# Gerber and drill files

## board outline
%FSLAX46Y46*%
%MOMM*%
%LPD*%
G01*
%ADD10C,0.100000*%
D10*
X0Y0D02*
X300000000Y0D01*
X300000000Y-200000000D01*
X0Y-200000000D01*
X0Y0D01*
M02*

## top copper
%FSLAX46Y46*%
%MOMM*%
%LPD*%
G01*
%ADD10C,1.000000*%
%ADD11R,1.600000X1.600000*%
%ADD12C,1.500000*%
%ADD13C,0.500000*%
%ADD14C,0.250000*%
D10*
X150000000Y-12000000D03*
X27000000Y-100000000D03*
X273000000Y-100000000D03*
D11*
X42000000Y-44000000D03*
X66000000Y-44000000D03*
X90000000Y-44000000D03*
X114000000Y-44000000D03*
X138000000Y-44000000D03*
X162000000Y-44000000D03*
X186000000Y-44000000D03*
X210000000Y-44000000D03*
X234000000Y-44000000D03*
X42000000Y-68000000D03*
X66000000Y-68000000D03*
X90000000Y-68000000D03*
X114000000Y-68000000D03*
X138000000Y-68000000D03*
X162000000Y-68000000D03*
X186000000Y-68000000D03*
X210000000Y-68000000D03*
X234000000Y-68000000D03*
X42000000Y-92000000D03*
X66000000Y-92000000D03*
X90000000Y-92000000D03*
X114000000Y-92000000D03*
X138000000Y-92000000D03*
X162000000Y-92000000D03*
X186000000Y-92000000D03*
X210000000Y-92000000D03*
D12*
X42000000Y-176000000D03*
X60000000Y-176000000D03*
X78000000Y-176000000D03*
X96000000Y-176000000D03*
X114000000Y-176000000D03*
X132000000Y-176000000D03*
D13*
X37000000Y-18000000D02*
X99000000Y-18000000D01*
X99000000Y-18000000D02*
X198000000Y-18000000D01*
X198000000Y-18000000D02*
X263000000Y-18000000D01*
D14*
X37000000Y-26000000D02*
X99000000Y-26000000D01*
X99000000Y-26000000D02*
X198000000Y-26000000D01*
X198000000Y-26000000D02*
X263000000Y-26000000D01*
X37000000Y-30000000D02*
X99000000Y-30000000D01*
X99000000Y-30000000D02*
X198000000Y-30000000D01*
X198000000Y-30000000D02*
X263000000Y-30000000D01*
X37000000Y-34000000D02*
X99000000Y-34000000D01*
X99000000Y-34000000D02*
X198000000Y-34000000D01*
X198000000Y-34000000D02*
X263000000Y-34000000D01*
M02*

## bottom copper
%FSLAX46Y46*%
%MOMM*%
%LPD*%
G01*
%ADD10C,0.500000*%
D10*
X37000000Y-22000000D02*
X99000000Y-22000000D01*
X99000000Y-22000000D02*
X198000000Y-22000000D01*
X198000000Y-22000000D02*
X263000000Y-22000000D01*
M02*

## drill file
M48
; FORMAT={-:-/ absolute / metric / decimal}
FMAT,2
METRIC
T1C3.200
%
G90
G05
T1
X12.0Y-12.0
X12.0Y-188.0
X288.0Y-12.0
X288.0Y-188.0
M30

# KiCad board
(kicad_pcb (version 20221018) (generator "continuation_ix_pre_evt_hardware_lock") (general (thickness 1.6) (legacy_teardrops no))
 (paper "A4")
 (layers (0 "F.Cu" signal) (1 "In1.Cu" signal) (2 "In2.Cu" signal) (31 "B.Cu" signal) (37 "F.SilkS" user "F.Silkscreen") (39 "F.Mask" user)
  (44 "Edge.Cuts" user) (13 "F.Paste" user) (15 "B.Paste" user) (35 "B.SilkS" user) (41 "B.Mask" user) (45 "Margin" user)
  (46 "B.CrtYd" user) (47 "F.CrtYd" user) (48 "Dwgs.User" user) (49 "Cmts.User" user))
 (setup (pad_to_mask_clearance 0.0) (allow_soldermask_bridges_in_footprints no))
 (gr_rect (start 0 0) (end 300.0 200.0) (stroke (width 0.1) (type default)) (fill none) (layer "Edge.Cuts"))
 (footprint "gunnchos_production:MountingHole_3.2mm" (layer "F.Cu") (at 12.0 12.0)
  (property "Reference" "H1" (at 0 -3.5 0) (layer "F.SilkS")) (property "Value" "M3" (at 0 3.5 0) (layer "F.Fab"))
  (pad "" np_thru_hole circle (at 0 0) (size 3.2 3.2) (drill 3.2) (layers "*.Cu" "*.Mask")))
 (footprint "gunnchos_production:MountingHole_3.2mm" (layer "F.Cu") (at 288.0 12.0)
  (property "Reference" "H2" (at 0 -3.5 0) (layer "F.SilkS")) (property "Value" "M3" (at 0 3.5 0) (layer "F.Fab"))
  (pad "" np_thru_hole circle (at 0 0) (size 3.2 3.2) (drill 3.2) (layers "*.Cu" "*.Mask")))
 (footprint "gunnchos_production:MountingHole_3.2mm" (layer "F.Cu") (at 12.0 188.0)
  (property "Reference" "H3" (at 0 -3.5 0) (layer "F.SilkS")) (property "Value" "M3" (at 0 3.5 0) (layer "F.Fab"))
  (pad "" np_thru_hole circle (at 0 0) (size 3.2 3.2) (drill 3.2) (layers "*.Cu" "*.Mask")))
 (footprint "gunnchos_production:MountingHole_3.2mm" (layer "F.Cu") (at 288.0 188.0)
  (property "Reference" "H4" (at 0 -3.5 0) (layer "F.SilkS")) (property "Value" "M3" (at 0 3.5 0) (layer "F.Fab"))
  (pad "" np_thru_hole circle (at 0 0) (size 3.2 3.2) (drill 3.2) (layers "*.Cu" "*.Mask")))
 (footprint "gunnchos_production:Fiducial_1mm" (layer "F.Cu") (at 150.0 12.0)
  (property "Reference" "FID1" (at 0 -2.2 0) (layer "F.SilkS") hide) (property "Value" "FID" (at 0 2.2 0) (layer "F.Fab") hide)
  (pad "1" smd circle (at 0 0) (size 1 1) (layers "F.Cu") (solder_mask_margin 0.5)))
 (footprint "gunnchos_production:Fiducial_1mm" (layer "F.Cu") (at 27.0 100.0)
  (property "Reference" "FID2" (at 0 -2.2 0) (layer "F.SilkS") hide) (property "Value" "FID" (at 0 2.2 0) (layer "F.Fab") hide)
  (pad "1" smd circle (at 0 0) (size 1 1) (layers "F.Cu") (solder_mask_margin 0.5)))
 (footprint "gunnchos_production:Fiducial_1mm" (layer "F.Cu") (at 273.0 100.0)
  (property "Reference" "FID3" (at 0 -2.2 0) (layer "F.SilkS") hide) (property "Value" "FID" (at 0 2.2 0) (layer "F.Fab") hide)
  (pad "1" smd circle (at 0 0) (size 1 1) (layers "F.Cu") (solder_mask_margin 0.5)))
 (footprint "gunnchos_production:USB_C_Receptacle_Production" (layer "F.Cu") (at 42.00 44.00)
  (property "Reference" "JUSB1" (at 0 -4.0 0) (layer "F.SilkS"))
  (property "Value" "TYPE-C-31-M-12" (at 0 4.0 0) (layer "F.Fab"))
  (pad "1" smd rect (at 0 0) (size 1.6 1.6) (layers "F.Cu" "F.Paste" "F.Mask")))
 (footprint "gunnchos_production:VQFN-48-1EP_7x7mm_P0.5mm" (layer "F.Cu") (at 66.00 44.00)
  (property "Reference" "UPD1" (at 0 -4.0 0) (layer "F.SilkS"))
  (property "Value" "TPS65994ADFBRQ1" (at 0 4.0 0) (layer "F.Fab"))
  (pad "1" smd rect (at 0 0) (size 1.6 1.6) (layers "F.Cu" "F.Paste" "F.Mask")))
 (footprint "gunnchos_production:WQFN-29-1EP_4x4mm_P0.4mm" (layer "F.Cu") (at 90.00 44.00)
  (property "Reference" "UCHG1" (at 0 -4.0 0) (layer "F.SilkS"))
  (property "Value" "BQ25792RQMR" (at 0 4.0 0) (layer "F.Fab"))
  (pad "1" smd rect (at 0 0) (size 1.6 1.6) (layers "F.Cu" "F.Paste" "F.Mask")))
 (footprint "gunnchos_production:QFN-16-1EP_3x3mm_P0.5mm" (layer "F.Cu") (at 114.00 44.00)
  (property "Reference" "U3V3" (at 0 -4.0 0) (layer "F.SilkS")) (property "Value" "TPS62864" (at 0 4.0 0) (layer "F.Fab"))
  (pad "1" smd rect (at 0 0) (size 1.6 1.6) (layers "F.Cu" "F.Paste" "F.Mask")))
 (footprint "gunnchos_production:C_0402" (layer "F.Cu") (at 138.00 44.00) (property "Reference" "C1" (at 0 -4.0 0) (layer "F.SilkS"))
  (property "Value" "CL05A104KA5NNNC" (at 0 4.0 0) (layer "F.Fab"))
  (pad "1" smd rect (at 0 0) (size 1.6 1.6) (layers "F.Cu" "F.Paste" "F.Mask")))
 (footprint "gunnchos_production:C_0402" (layer "F.Cu") (at 162.00 44.00) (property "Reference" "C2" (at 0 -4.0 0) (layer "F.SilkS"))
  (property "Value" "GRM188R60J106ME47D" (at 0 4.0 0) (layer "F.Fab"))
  (pad "1" smd rect (at 0 0) (size 1.6 1.6) (layers "F.Cu" "F.Paste" "F.Mask")))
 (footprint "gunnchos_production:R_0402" (layer "F.Cu") (at 186.00 44.00) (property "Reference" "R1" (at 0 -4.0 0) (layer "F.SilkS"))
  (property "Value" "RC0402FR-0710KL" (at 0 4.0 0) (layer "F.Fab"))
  (pad "1" smd rect (at 0 0) (size 1.6 1.6) (layers "F.Cu" "F.Paste" "F.Mask")))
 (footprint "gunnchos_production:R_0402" (layer "F.Cu") (at 210.00 44.00) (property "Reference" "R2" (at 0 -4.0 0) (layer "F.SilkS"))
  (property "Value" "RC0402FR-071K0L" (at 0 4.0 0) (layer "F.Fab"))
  (pad "1" smd rect (at 0 0) (size 1.6 1.6) (layers "F.Cu" "F.Paste" "F.Mask")))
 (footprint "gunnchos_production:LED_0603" (layer "F.Cu") (at 234.00 44.00) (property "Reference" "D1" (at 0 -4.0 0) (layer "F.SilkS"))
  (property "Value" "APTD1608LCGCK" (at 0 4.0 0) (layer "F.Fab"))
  (pad "1" smd rect (at 0 0) (size 1.6 1.6) (layers "F.Cu" "F.Paste" "F.Mask")))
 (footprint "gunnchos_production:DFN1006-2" (layer "F.Cu") (at 42.00 68.00)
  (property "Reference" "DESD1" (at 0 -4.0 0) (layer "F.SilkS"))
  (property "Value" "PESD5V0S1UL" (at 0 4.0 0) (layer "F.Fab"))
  (pad "1" smd rect (at 0 0) (size 1.6 1.6) (layers "F.Cu" "F.Paste" "F.Mask")))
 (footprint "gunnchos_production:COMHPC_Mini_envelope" (layer "F.Cu") (at 66.00 68.00)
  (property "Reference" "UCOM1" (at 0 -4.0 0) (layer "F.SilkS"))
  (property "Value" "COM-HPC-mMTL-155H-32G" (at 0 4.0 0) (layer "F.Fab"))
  (pad "1" smd rect (at 0 0) (size 1.6 1.6) (layers "F.Cu" "F.Paste" "F.Mask")))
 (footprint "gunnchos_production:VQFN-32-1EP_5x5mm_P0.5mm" (layer "F.Cu") (at 90.00 68.00)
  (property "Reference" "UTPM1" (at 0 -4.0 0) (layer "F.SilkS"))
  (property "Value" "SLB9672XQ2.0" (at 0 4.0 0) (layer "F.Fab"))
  (pad "1" smd rect (at 0 0) (size 1.6 1.6) (layers "F.Cu" "F.Paste" "F.Mask")))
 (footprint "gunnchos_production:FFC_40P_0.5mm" (layer "F.Cu") (at 114.00 68.00)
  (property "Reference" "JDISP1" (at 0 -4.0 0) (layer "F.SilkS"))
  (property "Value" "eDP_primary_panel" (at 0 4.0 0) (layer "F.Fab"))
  (pad "1" smd rect (at 0 0) (size 1.6 1.6) (layers "F.Cu" "F.Paste" "F.Mask")))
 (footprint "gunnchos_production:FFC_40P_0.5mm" (layer "F.Cu") (at 138.00 68.00)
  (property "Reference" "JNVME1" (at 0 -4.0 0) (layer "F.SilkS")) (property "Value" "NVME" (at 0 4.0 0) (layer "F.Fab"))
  (pad "1" smd rect (at 0 0) (size 1.6 1.6) (layers "F.Cu" "F.Paste" "F.Mask")))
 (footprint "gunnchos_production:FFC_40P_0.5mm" (layer "F.Cu") (at 162.00 68.00)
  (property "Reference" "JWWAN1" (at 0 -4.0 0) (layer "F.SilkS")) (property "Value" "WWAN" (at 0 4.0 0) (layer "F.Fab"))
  (pad "1" smd rect (at 0 0) (size 1.6 1.6) (layers "F.Cu" "F.Paste" "F.Mask")))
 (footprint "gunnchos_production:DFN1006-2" (layer "F.Cu") (at 186.00 68.00)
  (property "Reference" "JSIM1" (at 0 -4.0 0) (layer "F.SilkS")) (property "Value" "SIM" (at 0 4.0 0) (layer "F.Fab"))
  (pad "1" smd rect (at 0 0) (size 1.6 1.6) (layers "F.Cu" "F.Paste" "F.Mask")))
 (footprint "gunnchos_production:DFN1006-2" (layer "F.Cu") (at 210.00 68.00)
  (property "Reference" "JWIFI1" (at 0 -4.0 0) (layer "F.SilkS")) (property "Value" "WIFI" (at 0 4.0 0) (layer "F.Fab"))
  (pad "1" smd rect (at 0 0) (size 1.6 1.6) (layers "F.Cu" "F.Paste" "F.Mask")))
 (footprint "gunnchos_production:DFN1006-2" (layer "F.Cu") (at 234.00 68.00)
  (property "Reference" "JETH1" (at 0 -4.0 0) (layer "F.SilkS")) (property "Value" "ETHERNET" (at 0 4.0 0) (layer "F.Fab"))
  (pad "1" smd rect (at 0 0) (size 1.6 1.6) (layers "F.Cu" "F.Paste" "F.Mask")))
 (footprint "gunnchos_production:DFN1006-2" (layer "F.Cu") (at 42.00 92.00)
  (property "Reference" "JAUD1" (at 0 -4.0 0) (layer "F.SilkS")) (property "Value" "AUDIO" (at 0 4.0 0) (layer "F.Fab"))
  (pad "1" smd rect (at 0 0) (size 1.6 1.6) (layers "F.Cu" "F.Paste" "F.Mask")))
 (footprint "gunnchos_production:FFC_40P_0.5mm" (layer "F.Cu") (at 66.00 92.00)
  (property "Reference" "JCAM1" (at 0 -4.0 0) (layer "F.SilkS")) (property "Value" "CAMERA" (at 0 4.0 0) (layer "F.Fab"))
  (pad "1" smd rect (at 0 0) (size 1.6 1.6) (layers "F.Cu" "F.Paste" "F.Mask")))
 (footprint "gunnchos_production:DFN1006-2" (layer "F.Cu") (at 90.00 92.00)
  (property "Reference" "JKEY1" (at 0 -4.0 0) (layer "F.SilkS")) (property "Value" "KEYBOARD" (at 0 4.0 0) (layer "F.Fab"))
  (pad "1" smd rect (at 0 0) (size 1.6 1.6) (layers "F.Cu" "F.Paste" "F.Mask")))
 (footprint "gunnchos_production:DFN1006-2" (layer "F.Cu") (at 114.00 92.00)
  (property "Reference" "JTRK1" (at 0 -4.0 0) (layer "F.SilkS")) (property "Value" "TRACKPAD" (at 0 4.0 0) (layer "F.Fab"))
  (pad "1" smd rect (at 0 0) (size 1.6 1.6) (layers "F.Cu" "F.Paste" "F.Mask")))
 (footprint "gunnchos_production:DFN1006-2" (layer "F.Cu") (at 138.00 92.00)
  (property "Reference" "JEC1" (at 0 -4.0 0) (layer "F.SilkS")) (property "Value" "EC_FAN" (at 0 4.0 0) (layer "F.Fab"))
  (pad "1" smd rect (at 0 0) (size 1.6 1.6) (layers "F.Cu" "F.Paste" "F.Mask")))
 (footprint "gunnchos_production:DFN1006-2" (layer "F.Cu") (at 162.00 92.00)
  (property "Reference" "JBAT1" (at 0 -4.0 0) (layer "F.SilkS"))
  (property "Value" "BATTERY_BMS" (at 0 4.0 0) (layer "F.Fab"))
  (pad "1" smd rect (at 0 0) (size 1.6 1.6) (layers "F.Cu" "F.Paste" "F.Mask")))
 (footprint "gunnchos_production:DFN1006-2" (layer "F.Cu") (at 186.00 92.00)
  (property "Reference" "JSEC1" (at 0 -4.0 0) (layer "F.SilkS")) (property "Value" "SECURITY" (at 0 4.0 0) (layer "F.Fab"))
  (pad "1" smd rect (at 0 0) (size 1.6 1.6) (layers "F.Cu" "F.Paste" "F.Mask")))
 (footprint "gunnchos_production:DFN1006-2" (layer "F.Cu") (at 210.00 92.00)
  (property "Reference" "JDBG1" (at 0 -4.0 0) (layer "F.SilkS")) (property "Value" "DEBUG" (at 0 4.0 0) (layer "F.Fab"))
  (pad "1" smd rect (at 0 0) (size 1.6 1.6) (layers "F.Cu" "F.Paste" "F.Mask")))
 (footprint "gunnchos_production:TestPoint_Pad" (layer "F.Cu") (at 42.0 176.0) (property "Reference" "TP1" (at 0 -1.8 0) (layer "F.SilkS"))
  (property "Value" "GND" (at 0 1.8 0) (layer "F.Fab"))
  (pad "1" smd circle (at 0 0) (size 1.5 1.5) (layers "F.Cu" "F.Mask")))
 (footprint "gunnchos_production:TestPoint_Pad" (layer "F.Cu") (at 60.0 176.0) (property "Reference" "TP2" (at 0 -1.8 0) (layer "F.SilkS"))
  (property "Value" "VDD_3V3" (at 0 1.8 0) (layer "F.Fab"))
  (pad "1" smd circle (at 0 0) (size 1.5 1.5) (layers "F.Cu" "F.Mask")))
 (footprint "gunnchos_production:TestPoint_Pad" (layer "F.Cu") (at 78.0 176.0) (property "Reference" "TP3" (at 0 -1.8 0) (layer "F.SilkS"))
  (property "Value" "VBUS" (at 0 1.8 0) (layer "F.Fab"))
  (pad "1" smd circle (at 0 0) (size 1.5 1.5) (layers "F.Cu" "F.Mask")))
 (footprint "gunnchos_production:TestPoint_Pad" (layer "F.Cu") (at 96.0 176.0) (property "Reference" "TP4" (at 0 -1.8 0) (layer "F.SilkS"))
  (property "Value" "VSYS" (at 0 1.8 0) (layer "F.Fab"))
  (pad "1" smd circle (at 0 0) (size 1.5 1.5) (layers "F.Cu" "F.Mask")))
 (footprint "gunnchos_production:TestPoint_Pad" (layer "F.Cu") (at 114.0 176.0) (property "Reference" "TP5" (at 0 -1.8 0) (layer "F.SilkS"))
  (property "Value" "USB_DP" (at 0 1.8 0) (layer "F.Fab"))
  (pad "1" smd circle (at 0 0) (size 1.5 1.5) (layers "F.Cu" "F.Mask")))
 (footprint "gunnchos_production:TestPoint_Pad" (layer "F.Cu") (at 132.0 176.0) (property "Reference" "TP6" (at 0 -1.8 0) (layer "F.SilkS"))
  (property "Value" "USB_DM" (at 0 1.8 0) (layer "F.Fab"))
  (pad "1" smd circle (at 0 0) (size 1.5 1.5) (layers "F.Cu" "F.Mask")))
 (segment (start 37.00 18.00) (end 99.00 18.00) (width 0.5) (layer "F.Cu") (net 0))
 (segment (start 99.00 18.00) (end 198.00 18.00) (width 0.5) (layer "F.Cu") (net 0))
 (segment (start 198.00 18.00) (end 263.00 18.00) (width 0.5) (layer "F.Cu") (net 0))
 (segment (start 37.00 22.00) (end 99.00 22.00) (width 0.5) (layer "B.Cu") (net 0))
 (segment (start 99.00 22.00) (end 198.00 22.00) (width 0.5) (layer "B.Cu") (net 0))
 (segment (start 198.00 22.00) (end 263.00 22.00) (width 0.5) (layer "B.Cu") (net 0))
 (segment (start 37.00 26.00) (end 99.00 26.00) (width 0.25) (layer "F.Cu") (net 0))
 (segment (start 99.00 26.00) (end 198.00 26.00) (width 0.25) (layer "F.Cu") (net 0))
 (segment (start 198.00 26.00) (end 263.00 26.00) (width 0.25) (layer "F.Cu") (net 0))
 (segment (start 37.00 30.00) (end 99.00 30.00) (width 0.25) (layer "F.Cu") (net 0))
 (segment (start 99.00 30.00) (end 198.00 30.00) (width 0.25) (layer "F.Cu") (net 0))
 (segment (start 198.00 30.00) (end 263.00 30.00) (width 0.25) (layer "F.Cu") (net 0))
 (segment (start 37.00 34.00) (end 99.00 34.00) (width 0.25) (layer "F.Cu") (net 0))
 (segment (start 99.00 34.00) (end 198.00 34.00) (width 0.25) (layer "F.Cu") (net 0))
 (segment (start 198.00 34.00) (end 263.00 34.00) (width 0.25) (layer "F.Cu") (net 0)))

